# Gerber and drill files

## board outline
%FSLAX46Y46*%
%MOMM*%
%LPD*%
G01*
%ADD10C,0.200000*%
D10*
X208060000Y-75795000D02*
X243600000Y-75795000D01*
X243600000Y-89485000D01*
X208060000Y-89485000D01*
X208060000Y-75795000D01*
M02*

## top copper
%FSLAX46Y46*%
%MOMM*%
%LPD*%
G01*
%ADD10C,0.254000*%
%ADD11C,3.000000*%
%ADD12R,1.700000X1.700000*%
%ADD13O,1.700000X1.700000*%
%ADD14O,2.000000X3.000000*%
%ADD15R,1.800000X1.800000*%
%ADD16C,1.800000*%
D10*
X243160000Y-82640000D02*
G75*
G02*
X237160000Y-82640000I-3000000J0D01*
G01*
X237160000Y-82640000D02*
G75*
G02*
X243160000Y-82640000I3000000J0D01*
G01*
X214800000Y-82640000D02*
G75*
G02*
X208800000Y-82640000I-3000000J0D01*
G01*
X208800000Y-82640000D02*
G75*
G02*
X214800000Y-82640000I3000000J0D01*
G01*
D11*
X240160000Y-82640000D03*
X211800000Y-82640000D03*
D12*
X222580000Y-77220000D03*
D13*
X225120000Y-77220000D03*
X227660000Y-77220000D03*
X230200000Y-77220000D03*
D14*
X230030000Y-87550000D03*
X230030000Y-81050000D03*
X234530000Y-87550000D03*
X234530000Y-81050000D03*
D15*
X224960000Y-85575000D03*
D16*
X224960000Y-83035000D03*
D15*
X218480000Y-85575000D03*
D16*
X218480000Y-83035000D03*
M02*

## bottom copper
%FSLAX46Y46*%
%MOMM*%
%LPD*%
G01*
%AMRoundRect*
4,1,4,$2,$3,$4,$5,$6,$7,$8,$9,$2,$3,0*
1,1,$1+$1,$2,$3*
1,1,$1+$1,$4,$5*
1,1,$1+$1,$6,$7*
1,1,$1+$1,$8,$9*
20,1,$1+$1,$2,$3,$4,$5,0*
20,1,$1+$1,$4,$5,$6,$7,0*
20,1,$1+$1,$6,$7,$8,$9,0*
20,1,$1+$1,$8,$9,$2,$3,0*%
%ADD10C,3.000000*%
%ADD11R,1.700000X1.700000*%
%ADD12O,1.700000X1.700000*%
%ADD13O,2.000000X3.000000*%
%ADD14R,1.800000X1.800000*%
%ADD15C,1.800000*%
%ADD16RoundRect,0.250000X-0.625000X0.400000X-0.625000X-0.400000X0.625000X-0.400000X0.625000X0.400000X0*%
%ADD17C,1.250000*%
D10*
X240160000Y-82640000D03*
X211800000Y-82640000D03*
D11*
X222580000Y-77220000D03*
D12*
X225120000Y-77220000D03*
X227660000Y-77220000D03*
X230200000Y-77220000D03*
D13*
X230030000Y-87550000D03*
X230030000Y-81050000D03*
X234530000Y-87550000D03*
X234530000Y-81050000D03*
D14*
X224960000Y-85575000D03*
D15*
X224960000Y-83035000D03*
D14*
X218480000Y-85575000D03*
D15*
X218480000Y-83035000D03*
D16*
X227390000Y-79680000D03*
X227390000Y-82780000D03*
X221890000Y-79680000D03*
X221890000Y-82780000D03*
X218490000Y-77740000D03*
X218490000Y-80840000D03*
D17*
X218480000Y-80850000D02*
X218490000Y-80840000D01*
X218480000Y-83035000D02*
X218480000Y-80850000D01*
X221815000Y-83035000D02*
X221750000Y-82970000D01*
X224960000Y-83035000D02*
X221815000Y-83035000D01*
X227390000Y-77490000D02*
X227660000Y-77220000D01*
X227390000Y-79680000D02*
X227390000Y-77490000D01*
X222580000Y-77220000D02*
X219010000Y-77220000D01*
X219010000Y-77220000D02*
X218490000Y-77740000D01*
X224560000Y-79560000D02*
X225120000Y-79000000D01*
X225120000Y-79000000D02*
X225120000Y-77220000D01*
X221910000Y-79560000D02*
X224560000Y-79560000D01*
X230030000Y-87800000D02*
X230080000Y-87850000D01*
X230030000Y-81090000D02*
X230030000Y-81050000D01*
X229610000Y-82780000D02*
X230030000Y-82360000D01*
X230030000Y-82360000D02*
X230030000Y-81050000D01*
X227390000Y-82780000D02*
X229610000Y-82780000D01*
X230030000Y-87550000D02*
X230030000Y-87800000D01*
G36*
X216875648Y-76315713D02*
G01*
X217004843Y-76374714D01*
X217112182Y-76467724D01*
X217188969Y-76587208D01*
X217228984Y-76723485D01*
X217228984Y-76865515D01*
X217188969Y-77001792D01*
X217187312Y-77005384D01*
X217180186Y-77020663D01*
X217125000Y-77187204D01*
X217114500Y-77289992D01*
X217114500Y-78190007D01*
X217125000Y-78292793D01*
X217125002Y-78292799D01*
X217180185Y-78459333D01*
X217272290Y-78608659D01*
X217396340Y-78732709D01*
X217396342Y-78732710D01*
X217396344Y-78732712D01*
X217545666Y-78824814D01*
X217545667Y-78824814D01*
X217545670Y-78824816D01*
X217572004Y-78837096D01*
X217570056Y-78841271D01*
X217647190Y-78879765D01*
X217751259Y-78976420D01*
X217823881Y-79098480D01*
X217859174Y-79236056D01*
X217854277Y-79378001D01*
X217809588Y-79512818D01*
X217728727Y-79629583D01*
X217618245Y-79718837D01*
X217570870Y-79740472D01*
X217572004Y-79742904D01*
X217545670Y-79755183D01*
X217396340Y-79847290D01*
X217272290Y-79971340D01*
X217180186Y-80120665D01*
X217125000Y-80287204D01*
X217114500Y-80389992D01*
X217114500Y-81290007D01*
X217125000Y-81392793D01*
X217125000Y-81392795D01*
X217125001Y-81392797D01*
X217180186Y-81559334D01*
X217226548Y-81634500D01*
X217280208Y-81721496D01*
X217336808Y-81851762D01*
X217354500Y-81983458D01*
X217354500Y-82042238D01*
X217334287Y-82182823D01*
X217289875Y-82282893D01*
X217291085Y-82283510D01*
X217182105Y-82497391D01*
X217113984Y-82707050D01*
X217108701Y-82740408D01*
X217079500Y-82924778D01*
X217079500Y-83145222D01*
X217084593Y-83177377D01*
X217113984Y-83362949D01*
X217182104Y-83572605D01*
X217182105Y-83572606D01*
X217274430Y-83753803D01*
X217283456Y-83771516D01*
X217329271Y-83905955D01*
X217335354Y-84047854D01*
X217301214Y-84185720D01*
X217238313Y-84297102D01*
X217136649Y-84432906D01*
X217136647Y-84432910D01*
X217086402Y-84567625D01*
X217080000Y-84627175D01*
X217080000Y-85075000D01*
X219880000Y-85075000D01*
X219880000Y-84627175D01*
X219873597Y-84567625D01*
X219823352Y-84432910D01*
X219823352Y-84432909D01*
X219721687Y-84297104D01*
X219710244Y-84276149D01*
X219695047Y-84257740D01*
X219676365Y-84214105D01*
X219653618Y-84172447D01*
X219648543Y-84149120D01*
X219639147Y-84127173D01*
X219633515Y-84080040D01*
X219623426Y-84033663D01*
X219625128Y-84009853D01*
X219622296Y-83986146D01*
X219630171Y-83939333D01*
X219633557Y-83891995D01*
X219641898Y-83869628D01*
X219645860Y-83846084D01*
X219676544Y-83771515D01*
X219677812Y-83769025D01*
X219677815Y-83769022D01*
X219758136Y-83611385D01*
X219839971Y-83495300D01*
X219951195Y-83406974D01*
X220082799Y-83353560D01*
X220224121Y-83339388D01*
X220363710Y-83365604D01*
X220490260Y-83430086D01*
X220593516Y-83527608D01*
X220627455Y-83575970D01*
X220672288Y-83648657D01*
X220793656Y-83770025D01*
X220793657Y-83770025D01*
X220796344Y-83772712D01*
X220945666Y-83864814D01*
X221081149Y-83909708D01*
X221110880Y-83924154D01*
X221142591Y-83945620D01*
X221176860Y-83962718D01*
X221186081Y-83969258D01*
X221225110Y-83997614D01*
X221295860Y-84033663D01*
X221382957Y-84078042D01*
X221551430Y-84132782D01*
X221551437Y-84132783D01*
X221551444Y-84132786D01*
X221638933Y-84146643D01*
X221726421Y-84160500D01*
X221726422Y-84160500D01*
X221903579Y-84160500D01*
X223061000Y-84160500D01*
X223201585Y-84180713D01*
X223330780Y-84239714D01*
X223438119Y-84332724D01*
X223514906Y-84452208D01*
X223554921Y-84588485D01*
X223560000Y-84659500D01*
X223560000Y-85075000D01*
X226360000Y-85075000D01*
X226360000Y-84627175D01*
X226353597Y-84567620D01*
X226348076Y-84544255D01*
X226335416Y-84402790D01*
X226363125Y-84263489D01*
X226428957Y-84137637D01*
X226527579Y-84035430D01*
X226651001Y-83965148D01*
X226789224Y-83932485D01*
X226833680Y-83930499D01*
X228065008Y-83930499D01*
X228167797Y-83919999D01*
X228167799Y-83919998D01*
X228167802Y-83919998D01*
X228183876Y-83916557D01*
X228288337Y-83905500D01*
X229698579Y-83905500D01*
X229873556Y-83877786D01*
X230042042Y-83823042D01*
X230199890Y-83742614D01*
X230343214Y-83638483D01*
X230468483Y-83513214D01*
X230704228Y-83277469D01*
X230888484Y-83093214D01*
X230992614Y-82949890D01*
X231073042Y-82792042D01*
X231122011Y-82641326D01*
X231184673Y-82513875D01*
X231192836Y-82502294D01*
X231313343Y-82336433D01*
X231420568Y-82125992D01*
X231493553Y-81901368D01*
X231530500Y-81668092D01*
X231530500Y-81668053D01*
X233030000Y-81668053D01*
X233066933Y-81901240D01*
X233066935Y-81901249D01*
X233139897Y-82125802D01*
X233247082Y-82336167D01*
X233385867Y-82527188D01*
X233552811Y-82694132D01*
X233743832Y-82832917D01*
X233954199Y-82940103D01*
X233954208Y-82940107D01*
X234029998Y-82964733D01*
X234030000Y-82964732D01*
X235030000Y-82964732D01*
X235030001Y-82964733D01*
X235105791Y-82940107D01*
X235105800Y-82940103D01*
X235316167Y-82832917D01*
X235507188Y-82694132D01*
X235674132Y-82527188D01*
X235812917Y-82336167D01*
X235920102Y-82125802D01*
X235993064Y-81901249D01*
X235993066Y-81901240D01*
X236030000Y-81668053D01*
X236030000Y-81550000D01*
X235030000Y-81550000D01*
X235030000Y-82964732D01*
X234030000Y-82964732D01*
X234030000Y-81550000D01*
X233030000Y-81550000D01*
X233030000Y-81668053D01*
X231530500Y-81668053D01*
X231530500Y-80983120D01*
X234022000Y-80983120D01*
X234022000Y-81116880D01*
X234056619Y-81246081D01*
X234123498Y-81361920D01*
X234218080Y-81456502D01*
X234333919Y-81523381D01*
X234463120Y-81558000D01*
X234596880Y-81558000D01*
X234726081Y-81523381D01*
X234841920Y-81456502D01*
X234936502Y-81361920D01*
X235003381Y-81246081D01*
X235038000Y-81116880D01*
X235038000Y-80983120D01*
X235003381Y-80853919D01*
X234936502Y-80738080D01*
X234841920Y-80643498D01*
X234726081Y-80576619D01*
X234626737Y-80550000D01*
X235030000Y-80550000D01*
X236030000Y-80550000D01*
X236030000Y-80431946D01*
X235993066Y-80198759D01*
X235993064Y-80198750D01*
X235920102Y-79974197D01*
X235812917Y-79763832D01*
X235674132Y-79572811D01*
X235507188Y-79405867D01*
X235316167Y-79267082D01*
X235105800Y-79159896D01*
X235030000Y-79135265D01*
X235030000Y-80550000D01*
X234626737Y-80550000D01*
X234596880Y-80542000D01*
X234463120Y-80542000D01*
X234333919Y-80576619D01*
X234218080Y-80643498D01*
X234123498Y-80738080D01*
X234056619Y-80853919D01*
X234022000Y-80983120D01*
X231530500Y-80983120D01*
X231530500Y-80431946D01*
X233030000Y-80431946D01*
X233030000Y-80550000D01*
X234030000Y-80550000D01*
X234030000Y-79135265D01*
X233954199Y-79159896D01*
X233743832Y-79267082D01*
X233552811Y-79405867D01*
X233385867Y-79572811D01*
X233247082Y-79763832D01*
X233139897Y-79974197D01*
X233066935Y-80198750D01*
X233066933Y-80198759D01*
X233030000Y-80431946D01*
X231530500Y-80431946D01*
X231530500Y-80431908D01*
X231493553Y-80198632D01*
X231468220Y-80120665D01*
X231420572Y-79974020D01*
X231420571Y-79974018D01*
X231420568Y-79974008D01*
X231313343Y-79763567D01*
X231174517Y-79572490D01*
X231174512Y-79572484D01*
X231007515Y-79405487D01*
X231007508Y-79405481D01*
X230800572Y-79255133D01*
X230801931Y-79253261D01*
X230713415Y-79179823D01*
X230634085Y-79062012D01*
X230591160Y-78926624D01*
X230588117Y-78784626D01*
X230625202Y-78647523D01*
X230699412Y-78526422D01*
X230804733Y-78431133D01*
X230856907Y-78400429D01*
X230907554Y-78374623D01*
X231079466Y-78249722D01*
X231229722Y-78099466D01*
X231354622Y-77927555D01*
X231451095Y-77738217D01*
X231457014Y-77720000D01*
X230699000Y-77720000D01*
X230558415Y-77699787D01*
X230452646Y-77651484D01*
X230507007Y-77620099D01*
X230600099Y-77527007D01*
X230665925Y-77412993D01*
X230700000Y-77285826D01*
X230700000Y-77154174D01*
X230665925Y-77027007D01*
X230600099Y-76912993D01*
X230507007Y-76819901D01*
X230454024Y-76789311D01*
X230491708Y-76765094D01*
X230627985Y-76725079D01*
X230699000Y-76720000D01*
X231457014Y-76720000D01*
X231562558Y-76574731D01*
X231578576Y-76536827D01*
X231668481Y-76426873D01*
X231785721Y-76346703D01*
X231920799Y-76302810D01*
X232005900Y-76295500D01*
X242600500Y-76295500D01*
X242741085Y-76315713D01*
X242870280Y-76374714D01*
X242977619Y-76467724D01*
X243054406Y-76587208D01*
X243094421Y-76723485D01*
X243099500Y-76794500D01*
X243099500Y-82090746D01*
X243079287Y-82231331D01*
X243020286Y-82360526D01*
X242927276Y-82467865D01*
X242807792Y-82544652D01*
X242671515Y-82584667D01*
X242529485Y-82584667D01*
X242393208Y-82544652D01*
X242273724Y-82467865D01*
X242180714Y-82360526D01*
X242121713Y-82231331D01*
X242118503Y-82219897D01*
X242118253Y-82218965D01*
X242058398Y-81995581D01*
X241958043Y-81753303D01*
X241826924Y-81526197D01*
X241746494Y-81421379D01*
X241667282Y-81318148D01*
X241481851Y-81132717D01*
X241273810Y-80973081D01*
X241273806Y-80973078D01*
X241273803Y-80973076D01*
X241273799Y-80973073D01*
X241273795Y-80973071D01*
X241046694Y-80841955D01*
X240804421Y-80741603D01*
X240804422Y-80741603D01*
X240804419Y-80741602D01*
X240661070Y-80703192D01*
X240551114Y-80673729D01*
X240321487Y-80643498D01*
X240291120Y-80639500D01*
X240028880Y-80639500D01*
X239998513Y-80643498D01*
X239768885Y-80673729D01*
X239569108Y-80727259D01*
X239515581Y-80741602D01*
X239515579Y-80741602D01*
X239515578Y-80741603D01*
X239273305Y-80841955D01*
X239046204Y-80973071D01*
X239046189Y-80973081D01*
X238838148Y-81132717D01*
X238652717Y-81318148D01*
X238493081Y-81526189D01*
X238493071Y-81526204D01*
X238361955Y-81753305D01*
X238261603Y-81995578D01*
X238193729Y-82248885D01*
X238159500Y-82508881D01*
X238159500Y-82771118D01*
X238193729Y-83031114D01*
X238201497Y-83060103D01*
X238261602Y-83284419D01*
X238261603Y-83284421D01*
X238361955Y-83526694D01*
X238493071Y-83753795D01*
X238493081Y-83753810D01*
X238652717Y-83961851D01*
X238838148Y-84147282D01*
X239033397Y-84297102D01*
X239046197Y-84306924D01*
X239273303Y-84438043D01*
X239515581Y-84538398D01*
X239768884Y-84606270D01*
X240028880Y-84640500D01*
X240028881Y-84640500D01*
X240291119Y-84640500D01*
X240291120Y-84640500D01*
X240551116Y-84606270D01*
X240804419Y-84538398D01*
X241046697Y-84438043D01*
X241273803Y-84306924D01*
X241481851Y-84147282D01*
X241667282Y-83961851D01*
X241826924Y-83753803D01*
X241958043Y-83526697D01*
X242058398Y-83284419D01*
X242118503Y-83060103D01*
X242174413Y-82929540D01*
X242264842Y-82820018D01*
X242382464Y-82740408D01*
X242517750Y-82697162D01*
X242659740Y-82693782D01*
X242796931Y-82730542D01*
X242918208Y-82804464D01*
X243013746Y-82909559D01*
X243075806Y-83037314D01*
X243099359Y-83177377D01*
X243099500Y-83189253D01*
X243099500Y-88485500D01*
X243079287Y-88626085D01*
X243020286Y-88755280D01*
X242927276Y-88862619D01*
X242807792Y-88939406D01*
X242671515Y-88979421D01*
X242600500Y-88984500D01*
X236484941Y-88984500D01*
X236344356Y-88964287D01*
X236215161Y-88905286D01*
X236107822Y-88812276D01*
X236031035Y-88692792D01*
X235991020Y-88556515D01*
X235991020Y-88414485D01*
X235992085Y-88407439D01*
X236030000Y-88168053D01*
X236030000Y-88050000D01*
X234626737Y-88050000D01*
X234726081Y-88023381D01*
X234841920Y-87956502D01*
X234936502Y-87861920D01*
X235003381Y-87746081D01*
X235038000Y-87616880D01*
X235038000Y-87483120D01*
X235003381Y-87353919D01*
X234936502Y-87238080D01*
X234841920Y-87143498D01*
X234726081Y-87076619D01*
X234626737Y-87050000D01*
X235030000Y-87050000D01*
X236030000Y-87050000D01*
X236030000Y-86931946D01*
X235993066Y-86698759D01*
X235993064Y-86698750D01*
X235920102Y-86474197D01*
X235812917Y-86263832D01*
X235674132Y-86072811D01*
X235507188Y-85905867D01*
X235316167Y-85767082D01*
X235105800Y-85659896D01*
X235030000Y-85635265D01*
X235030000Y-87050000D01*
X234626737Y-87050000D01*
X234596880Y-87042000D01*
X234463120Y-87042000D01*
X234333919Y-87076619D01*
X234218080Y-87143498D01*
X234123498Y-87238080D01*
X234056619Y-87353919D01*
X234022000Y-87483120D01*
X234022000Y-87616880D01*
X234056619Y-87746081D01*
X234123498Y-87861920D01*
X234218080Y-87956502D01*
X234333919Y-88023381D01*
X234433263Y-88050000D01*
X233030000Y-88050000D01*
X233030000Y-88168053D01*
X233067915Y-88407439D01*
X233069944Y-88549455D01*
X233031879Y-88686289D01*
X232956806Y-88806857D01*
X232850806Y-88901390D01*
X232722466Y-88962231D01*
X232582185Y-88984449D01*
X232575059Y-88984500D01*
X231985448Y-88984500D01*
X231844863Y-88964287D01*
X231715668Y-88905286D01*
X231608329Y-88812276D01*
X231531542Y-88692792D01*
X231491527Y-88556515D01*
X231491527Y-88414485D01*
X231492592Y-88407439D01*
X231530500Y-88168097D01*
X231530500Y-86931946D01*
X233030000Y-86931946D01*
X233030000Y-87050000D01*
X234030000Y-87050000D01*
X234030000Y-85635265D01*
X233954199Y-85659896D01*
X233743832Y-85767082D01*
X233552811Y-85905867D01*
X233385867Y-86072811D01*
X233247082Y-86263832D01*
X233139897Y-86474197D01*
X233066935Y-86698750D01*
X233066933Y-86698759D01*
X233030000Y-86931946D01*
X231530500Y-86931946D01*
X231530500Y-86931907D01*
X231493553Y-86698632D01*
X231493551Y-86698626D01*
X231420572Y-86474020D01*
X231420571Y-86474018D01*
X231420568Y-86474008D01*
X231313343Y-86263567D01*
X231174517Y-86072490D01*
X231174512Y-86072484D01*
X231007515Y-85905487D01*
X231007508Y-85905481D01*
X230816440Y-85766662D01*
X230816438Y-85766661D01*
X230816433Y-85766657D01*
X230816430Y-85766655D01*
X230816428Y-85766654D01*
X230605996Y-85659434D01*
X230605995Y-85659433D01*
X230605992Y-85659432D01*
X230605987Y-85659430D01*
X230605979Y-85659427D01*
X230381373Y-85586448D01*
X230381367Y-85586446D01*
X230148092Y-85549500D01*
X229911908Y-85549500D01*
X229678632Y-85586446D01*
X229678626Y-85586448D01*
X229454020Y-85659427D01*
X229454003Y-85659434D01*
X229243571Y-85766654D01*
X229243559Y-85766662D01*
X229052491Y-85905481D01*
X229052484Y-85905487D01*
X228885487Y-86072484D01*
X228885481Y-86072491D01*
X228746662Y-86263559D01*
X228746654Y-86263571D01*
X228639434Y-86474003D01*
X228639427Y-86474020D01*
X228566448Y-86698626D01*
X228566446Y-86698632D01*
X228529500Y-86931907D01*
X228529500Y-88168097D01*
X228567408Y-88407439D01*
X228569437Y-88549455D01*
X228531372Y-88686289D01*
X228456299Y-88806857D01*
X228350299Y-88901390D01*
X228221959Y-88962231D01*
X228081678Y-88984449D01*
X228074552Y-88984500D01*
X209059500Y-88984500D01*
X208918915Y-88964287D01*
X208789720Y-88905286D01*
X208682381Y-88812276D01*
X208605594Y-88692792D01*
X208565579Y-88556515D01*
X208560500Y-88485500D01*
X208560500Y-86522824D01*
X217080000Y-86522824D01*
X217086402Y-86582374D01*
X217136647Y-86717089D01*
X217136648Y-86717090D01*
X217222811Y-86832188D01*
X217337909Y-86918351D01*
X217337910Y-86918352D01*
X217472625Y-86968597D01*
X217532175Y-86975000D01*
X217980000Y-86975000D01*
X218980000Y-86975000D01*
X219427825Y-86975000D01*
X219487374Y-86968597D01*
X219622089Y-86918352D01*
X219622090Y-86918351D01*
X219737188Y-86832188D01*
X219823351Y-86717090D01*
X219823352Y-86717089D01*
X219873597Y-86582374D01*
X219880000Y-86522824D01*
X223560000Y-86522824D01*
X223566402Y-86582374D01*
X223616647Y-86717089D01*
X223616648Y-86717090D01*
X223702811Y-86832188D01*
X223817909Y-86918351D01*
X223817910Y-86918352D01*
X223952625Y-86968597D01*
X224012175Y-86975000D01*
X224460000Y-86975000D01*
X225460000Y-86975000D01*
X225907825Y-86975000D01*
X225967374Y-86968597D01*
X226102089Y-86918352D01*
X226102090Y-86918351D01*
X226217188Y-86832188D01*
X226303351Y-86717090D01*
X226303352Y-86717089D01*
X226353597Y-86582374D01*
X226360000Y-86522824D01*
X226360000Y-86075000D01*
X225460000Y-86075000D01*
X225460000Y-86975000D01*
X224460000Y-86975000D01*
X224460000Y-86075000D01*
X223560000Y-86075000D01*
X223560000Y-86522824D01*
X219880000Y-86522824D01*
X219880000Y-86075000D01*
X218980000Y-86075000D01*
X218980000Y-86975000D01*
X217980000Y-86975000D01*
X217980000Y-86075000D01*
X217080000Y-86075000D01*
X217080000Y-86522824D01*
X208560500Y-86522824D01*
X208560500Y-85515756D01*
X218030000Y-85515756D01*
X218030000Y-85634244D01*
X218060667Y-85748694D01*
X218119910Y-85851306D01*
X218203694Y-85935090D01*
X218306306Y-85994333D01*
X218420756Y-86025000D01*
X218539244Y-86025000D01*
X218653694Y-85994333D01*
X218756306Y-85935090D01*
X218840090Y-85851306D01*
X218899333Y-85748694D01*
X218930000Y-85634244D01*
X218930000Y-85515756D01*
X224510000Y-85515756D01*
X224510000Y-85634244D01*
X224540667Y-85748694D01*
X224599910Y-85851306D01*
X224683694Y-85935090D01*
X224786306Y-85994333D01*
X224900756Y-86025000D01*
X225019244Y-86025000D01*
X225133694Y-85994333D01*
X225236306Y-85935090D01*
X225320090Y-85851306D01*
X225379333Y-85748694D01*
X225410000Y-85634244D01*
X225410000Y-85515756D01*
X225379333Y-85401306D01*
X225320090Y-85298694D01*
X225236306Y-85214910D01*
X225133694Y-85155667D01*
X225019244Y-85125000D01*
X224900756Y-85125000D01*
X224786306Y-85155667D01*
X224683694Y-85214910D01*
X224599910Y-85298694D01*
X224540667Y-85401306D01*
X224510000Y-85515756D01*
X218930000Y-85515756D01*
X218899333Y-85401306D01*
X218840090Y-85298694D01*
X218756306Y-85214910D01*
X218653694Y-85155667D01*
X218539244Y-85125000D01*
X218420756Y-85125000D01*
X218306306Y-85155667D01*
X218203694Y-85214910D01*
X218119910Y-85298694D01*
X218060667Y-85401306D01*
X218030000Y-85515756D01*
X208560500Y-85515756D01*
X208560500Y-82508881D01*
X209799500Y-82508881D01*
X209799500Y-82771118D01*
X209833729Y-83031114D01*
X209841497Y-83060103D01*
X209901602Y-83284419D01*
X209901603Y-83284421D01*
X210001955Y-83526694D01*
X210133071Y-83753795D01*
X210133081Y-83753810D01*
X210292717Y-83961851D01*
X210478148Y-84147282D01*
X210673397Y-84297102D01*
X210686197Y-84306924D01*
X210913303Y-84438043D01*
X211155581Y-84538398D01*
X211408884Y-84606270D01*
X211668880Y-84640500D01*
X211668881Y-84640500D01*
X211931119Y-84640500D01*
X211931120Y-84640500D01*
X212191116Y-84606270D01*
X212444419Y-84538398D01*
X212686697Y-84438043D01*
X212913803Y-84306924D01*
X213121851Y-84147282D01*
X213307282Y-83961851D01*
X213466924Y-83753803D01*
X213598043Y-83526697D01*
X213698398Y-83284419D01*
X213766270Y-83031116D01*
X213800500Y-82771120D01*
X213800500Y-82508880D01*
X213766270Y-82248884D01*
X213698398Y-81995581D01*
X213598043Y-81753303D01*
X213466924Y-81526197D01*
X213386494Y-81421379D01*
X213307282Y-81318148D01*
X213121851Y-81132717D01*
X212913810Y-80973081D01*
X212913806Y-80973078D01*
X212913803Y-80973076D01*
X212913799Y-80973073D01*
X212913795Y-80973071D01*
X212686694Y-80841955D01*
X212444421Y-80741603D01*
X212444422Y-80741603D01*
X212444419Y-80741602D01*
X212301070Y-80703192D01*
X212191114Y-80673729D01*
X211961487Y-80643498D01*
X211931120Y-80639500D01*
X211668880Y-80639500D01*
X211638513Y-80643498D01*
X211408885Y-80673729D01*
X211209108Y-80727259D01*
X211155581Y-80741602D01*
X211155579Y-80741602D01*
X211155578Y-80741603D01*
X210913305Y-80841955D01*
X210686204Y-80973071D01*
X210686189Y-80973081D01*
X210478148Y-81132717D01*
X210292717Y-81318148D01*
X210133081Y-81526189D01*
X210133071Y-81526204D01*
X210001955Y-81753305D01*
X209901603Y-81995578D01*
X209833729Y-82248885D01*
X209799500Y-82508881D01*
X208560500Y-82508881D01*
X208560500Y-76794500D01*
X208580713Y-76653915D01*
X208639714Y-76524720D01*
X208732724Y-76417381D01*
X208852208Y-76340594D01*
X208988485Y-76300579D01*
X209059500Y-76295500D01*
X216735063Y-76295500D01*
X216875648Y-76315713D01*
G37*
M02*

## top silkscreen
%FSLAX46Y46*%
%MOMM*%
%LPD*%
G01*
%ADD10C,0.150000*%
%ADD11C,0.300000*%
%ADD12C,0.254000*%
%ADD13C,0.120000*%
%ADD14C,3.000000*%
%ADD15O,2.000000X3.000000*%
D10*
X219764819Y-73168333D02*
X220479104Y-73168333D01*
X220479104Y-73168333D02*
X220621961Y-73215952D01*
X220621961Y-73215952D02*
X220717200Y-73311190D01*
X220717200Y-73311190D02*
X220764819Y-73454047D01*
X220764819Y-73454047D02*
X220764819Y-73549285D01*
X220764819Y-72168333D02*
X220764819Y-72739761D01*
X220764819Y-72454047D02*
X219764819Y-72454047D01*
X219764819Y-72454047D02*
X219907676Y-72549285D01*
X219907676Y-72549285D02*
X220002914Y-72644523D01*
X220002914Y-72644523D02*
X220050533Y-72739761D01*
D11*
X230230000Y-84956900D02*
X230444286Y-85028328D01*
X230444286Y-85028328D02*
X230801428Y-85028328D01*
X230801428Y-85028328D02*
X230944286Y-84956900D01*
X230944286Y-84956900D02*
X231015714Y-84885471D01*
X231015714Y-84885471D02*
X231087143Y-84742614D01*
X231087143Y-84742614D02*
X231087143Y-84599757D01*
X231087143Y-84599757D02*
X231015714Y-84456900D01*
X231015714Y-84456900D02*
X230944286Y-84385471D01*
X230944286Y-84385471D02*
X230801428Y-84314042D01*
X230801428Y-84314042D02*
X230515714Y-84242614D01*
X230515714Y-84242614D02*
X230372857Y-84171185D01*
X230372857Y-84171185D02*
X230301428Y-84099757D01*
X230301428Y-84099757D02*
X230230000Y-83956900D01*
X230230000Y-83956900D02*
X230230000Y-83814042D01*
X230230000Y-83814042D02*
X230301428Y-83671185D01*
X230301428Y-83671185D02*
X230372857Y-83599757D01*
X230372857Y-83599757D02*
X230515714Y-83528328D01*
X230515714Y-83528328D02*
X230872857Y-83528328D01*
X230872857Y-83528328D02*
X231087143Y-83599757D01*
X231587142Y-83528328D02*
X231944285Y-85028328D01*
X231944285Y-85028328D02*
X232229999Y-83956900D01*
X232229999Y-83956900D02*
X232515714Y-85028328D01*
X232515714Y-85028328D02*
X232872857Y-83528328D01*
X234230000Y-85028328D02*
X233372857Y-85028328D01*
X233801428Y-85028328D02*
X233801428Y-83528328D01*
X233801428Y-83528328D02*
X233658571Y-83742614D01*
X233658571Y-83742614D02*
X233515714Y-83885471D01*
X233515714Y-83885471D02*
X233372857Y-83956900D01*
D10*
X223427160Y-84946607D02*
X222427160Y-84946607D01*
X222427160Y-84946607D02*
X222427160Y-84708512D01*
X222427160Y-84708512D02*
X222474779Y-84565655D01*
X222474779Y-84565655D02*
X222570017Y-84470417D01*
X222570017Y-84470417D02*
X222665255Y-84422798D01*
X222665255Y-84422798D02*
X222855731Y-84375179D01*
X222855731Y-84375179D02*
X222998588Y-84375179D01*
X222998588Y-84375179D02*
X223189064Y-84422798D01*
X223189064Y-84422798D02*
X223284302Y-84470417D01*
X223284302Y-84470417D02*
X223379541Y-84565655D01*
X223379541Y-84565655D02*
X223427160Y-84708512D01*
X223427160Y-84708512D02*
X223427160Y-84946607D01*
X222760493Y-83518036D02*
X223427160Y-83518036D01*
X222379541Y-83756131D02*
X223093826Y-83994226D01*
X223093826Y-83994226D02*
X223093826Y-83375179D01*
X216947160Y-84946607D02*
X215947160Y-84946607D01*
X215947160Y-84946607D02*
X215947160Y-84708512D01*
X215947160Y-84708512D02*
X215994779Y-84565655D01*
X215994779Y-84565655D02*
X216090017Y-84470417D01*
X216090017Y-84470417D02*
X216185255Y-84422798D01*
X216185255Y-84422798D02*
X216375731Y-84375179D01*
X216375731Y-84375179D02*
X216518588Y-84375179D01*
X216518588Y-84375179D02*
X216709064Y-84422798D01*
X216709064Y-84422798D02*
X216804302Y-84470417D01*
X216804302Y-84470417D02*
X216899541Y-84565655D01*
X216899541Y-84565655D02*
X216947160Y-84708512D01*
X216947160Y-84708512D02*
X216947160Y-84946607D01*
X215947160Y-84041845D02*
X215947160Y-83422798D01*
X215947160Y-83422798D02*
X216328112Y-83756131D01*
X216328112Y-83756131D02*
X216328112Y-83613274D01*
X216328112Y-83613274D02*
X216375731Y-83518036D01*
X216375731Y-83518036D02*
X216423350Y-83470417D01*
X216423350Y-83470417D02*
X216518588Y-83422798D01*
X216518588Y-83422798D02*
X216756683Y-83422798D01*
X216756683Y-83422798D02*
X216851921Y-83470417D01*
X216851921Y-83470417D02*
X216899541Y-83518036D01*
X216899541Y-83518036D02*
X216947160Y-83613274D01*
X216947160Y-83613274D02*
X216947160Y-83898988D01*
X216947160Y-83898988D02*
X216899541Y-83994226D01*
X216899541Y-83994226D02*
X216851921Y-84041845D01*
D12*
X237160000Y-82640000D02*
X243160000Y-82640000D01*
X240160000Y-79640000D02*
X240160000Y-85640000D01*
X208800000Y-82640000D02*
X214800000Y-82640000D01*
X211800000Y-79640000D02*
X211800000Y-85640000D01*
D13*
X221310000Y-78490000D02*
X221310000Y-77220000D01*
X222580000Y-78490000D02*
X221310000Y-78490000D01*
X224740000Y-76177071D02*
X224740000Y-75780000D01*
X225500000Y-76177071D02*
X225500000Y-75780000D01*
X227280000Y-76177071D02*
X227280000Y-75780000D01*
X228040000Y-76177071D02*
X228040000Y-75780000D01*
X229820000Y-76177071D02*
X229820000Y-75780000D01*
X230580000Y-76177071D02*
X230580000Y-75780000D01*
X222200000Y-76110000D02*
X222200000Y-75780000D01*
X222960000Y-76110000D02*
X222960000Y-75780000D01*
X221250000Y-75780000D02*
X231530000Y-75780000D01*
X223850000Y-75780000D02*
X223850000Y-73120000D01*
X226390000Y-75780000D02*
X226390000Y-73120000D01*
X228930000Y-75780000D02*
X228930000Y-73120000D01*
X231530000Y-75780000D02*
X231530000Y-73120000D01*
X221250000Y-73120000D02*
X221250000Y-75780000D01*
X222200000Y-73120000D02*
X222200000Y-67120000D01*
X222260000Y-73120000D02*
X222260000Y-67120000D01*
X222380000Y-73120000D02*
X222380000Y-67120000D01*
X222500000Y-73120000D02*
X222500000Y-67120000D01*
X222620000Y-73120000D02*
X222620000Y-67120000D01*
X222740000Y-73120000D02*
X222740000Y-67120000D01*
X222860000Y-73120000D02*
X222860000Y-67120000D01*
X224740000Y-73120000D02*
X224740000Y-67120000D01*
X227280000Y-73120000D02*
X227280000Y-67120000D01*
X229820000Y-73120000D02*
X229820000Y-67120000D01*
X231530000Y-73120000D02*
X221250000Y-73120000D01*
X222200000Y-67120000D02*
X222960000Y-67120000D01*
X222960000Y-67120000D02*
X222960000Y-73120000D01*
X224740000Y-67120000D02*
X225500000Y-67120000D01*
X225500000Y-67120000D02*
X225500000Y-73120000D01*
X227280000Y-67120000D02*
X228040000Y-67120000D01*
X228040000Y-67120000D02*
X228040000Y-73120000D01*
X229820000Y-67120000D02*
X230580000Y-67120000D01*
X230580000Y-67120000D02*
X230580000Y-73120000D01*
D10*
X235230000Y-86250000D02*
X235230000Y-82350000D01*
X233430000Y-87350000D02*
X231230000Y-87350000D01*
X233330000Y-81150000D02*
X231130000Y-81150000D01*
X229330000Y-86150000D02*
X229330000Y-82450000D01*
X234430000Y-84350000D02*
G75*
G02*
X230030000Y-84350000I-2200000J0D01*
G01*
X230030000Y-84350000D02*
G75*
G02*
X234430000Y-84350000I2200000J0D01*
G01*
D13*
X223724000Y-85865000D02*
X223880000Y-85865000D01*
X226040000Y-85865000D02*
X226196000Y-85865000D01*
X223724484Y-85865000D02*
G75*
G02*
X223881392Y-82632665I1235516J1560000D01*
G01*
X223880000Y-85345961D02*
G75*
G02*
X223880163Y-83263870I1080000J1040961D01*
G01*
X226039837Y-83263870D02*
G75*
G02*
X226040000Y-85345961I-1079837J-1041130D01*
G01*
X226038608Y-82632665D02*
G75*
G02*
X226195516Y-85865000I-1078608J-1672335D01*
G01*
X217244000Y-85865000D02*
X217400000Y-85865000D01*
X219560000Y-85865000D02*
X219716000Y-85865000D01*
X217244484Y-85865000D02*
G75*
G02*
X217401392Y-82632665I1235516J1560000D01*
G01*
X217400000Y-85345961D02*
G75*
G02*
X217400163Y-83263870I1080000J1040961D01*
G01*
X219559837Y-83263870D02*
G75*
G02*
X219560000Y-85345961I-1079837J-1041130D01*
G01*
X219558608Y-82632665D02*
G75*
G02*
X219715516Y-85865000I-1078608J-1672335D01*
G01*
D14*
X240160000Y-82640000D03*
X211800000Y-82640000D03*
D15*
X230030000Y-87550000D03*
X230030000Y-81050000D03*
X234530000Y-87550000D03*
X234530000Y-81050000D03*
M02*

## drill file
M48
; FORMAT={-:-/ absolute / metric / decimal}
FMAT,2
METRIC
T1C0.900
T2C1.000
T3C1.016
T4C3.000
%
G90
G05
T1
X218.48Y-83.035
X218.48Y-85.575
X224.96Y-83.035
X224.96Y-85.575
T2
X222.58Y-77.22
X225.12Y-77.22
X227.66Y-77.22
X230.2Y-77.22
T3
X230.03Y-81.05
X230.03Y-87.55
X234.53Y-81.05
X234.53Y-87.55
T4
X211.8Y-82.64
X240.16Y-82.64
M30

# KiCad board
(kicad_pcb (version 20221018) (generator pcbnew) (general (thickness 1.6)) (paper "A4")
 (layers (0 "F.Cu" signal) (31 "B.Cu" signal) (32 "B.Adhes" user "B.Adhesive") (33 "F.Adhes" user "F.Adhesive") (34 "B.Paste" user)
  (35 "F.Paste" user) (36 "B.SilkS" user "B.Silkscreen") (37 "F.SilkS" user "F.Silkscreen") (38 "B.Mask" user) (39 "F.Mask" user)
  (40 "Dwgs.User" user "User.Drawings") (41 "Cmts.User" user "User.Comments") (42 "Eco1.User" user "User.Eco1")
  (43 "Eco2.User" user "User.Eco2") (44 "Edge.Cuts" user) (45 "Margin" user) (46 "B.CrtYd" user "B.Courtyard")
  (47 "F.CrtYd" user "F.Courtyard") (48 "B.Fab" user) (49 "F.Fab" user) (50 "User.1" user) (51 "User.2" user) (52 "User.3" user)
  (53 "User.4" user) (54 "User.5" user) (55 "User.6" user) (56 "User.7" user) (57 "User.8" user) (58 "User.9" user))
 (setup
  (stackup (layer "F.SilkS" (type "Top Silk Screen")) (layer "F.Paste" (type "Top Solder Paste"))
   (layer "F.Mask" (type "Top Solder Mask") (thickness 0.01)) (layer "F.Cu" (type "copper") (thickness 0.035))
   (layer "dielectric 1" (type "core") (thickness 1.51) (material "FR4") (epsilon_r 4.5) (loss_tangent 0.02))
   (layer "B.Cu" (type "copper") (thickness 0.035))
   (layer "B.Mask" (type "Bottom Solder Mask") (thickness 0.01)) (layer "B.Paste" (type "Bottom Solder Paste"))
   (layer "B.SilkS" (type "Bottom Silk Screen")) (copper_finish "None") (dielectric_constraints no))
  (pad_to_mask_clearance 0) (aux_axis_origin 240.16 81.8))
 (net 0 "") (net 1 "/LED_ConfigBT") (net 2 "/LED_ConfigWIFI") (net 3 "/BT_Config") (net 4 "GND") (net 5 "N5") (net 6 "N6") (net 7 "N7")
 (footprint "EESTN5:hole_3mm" (layer "F.Cu") (at 240.16 82.64)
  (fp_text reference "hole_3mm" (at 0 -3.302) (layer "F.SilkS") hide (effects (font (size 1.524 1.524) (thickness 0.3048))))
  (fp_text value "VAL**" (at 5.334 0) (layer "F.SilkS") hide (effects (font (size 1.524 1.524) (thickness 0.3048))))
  (fp_circle (center 0 0) (end 3 0) (stroke (width 0.254) (type solid)) (fill none) (layer "F.Cu"))
  (fp_line (start -3 0) (end 3 0) (stroke (width 0.254) (type solid)) (layer "F.SilkS"))
  (fp_line (start 0 -3) (end 0 3) (stroke (width 0.254) (type solid)) (layer "F.SilkS"))
  (pad "1" thru_hole circle (at 0 0) (size 3 3) (drill 3) (layers "*.Cu" "F.SilkS")))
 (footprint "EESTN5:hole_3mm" (layer "F.Cu") (at 211.8 82.64)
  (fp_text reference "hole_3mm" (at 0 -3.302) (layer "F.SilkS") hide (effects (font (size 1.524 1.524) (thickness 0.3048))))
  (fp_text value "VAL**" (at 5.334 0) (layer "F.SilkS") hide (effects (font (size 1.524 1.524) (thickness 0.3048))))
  (fp_circle (center 0 0) (end 3 0) (stroke (width 0.254) (type solid)) (fill none) (layer "F.Cu"))
  (fp_line (start -3 0) (end 3 0) (stroke (width 0.254) (type solid)) (layer "F.SilkS"))
  (fp_line (start 0 -3) (end 0 3) (stroke (width 0.254) (type solid)) (layer "F.SilkS"))
  (pad "1" thru_hole circle (at 0 0) (size 3 3) (drill 3) (layers "*.Cu" "F.SilkS")))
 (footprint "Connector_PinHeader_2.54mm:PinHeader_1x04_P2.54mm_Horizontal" (layer "F.Cu") (at 222.58 77.22 90)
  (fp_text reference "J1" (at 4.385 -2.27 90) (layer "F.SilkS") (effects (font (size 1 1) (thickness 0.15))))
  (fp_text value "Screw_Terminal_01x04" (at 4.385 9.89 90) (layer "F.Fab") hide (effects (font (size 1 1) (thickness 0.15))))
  (fp_line (start -1.27 -1.27) (end 0 -1.27) (stroke (width 0.12) (type solid)) (layer "F.SilkS"))
  (fp_line (start -1.27 0) (end -1.27 -1.27) (stroke (width 0.12) (type solid)) (layer "F.SilkS"))
  (fp_line (start 1.042929 2.16) (end 1.44 2.16) (stroke (width 0.12) (type solid)) (layer "F.SilkS"))
  (fp_line (start 1.042929 2.92) (end 1.44 2.92) (stroke (width 0.12) (type solid)) (layer "F.SilkS"))
  (fp_line (start 1.042929 4.7) (end 1.44 4.7) (stroke (width 0.12) (type solid)) (layer "F.SilkS"))
  (fp_line (start 1.042929 5.46) (end 1.44 5.46) (stroke (width 0.12) (type solid)) (layer "F.SilkS"))
  (fp_line (start 1.042929 7.24) (end 1.44 7.24) (stroke (width 0.12) (type solid)) (layer "F.SilkS"))
  (fp_line (start 1.042929 8) (end 1.44 8) (stroke (width 0.12) (type solid)) (layer "F.SilkS"))
  (fp_line (start 1.11 -0.38) (end 1.44 -0.38) (stroke (width 0.12) (type solid)) (layer "F.SilkS"))
  (fp_line (start 1.11 0.38) (end 1.44 0.38) (stroke (width 0.12) (type solid)) (layer "F.SilkS"))
  (fp_line (start 1.44 -1.33) (end 1.44 8.95) (stroke (width 0.12) (type solid)) (layer "F.SilkS"))
  (fp_line (start 1.44 1.27) (end 4.1 1.27) (stroke (width 0.12) (type solid)) (layer "F.SilkS"))
  (fp_line (start 1.44 3.81) (end 4.1 3.81) (stroke (width 0.12) (type solid)) (layer "F.SilkS"))
  (fp_line (start 1.44 6.35) (end 4.1 6.35) (stroke (width 0.12) (type solid)) (layer "F.SilkS"))
  (fp_line (start 1.44 8.95) (end 4.1 8.95) (stroke (width 0.12) (type solid)) (layer "F.SilkS"))
  (fp_line (start 4.1 -1.33) (end 1.44 -1.33) (stroke (width 0.12) (type solid)) (layer "F.SilkS"))
  (fp_line (start 4.1 -0.38) (end 10.1 -0.38) (stroke (width 0.12) (type solid)) (layer "F.SilkS"))
  (fp_line (start 4.1 -0.32) (end 10.1 -0.32) (stroke (width 0.12) (type solid)) (layer "F.SilkS"))
  (fp_line (start 4.1 -0.2) (end 10.1 -0.2) (stroke (width 0.12) (type solid)) (layer "F.SilkS"))
  (fp_line (start 4.1 -0.08) (end 10.1 -0.08) (stroke (width 0.12) (type solid)) (layer "F.SilkS"))
  (fp_line (start 4.1 0.04) (end 10.1 0.04) (stroke (width 0.12) (type solid)) (layer "F.SilkS"))
  (fp_line (start 4.1 0.16) (end 10.1 0.16) (stroke (width 0.12) (type solid)) (layer "F.SilkS"))
  (fp_line (start 4.1 0.28) (end 10.1 0.28) (stroke (width 0.12) (type solid)) (layer "F.SilkS"))
  (fp_line (start 4.1 2.16) (end 10.1 2.16) (stroke (width 0.12) (type solid)) (layer "F.SilkS"))
  (fp_line (start 4.1 4.7) (end 10.1 4.7) (stroke (width 0.12) (type solid)) (layer "F.SilkS"))
  (fp_line (start 4.1 7.24) (end 10.1 7.24) (stroke (width 0.12) (type solid)) (layer "F.SilkS"))
  (fp_line (start 4.1 8.95) (end 4.1 -1.33) (stroke (width 0.12) (type solid)) (layer "F.SilkS"))
  (fp_line (start 10.1 -0.38) (end 10.1 0.38) (stroke (width 0.12) (type solid)) (layer "F.SilkS"))
  (fp_line (start 10.1 0.38) (end 4.1 0.38) (stroke (width 0.12) (type solid)) (layer "F.SilkS"))
  (fp_line (start 10.1 2.16) (end 10.1 2.92) (stroke (width 0.12) (type solid)) (layer "F.SilkS"))
  (fp_line (start 10.1 2.92) (end 4.1 2.92) (stroke (width 0.12) (type solid)) (layer "F.SilkS"))
  (fp_line (start 10.1 4.7) (end 10.1 5.46) (stroke (width 0.12) (type solid)) (layer "F.SilkS"))
  (fp_line (start 10.1 5.46) (end 4.1 5.46) (stroke (width 0.12) (type solid)) (layer "F.SilkS"))
  (fp_line (start 10.1 7.24) (end 10.1 8) (stroke (width 0.12) (type solid)) (layer "F.SilkS"))
  (fp_line (start 10.1 8) (end 4.1 8) (stroke (width 0.12) (type solid)) (layer "F.SilkS"))
  (pad "1" thru_hole rect (at 0 0 90) (size 1.7 1.7) (drill 1) (layers "*.Cu" "*.Mask") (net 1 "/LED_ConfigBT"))
  (pad "2" thru_hole oval (at 0 2.54 90) (size 1.7 1.7) (drill 1) (layers "*.Cu" "*.Mask") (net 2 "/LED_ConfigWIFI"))
  (pad "3" thru_hole oval (at 0 5.08 90) (size 1.7 1.7) (drill 1) (layers "*.Cu" "*.Mask") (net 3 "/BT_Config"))
  (pad "4" thru_hole oval (at 0 7.62 90) (size 1.7 1.7) (drill 1) (layers "*.Cu" "*.Mask") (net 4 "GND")))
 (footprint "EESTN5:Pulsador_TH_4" (layer "F.Cu") (at 232.28 84.3 180)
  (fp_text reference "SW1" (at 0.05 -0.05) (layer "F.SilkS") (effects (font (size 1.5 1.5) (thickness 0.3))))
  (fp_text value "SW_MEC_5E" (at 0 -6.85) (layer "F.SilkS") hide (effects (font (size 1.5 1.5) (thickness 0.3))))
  (fp_line (start -2.95 -1.95) (end -2.95 1.95) (stroke (width 0.15) (type solid)) (layer "F.SilkS"))
  (fp_line (start -1.15 -3.05) (end 1.05 -3.05) (stroke (width 0.15) (type solid)) (layer "F.SilkS"))
  (fp_line (start -1.05 3.15) (end 1.15 3.15) (stroke (width 0.15) (type solid)) (layer "F.SilkS"))
  (fp_line (start 2.95 -1.85) (end 2.95 1.85) (stroke (width 0.15) (type solid)) (layer "F.SilkS"))
  (fp_circle (center 0.05 -0.05) (end 0.05 2.15) (stroke (width 0.15) (type solid)) (fill none) (layer "F.SilkS"))
  (pad "1" thru_hole oval (at 2.25 -3.25 180) (size 2 3) (drill 1.016) (layers "*.Cu" "*.Mask" "F.SilkS") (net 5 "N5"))
  (pad "2" thru_hole oval (at 2.25 3.25 180) (size 2 3) (drill 1.016) (layers "*.Cu" "*.Mask" "F.SilkS") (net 5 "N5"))
  (pad "3" thru_hole oval (at -2.25 -3.25 180) (size 2 3) (drill 1.016) (layers "*.Cu" "*.Mask" "F.SilkS") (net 4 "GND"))
  (pad "4" thru_hole oval (at -2.25 3.25 180) (size 2 3) (drill 1.016) (layers "*.Cu" "*.Mask" "F.SilkS") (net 4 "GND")))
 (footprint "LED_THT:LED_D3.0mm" (layer "F.Cu") (at 224.96 85.575 90)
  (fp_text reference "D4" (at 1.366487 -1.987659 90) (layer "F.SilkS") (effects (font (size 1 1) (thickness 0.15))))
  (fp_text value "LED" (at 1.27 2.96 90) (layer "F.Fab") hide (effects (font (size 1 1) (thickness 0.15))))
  (fp_line (start -0.29 -1.236) (end -0.29 -1.08) (stroke (width 0.12) (type solid)) (layer "F.SilkS"))
  (fp_line (start -0.29 1.08) (end -0.29 1.236) (stroke (width 0.12) (type solid)) (layer "F.SilkS"))
  (fp_arc (start -0.29 -1.235516) (mid 1.366487 -1.987659) (end 2.942335 -1.078608) (stroke (width 0.12) (type solid)) (layer "F.SilkS"))
  (fp_arc (start 0.229039 -1.08) (mid 1.270117 -1.5) (end 2.31113 -1.079837) (stroke (width 0.12) (type solid)) (layer "F.SilkS"))
  (fp_arc (start 2.31113 1.079837) (mid 1.270117 1.5) (end 0.229039 1.08) (stroke (width 0.12) (type solid)) (layer "F.SilkS"))
  (fp_arc (start 2.942335 1.078608) (mid 1.366487 1.987659) (end -0.29 1.235516) (stroke (width 0.12) (type solid)) (layer "F.SilkS"))
  (pad "1" thru_hole rect (at 0 0 90) (size 1.8 1.8) (drill 0.9) (layers "*.Cu" "*.Mask") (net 4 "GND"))
  (pad "2" thru_hole circle (at 2.54 0 90) (size 1.8 1.8) (drill 0.9) (layers "*.Cu" "*.Mask") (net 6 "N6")))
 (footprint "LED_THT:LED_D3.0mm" (layer "F.Cu") (at 218.48 85.575 90)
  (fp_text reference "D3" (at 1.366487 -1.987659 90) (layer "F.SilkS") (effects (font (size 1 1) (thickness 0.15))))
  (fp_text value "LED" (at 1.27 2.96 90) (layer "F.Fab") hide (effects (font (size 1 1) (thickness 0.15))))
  (fp_line (start -0.29 -1.236) (end -0.29 -1.08) (stroke (width 0.12) (type solid)) (layer "F.SilkS"))
  (fp_line (start -0.29 1.08) (end -0.29 1.236) (stroke (width 0.12) (type solid)) (layer "F.SilkS"))
  (fp_arc (start -0.29 -1.235516) (mid 1.366487 -1.987659) (end 2.942335 -1.078608) (stroke (width 0.12) (type solid)) (layer "F.SilkS"))
  (fp_arc (start 0.229039 -1.08) (mid 1.270117 -1.5) (end 2.31113 -1.079837) (stroke (width 0.12) (type solid)) (layer "F.SilkS"))
  (fp_arc (start 2.31113 1.079837) (mid 1.270117 1.5) (end 0.229039 1.08) (stroke (width 0.12) (type solid)) (layer "F.SilkS"))
  (fp_arc (start 2.942335 1.078608) (mid 1.366487 1.987659) (end -0.29 1.235516) (stroke (width 0.12) (type solid)) (layer "F.SilkS"))
  (pad "1" thru_hole rect (at 0 0 90) (size 1.8 1.8) (drill 0.9) (layers "*.Cu" "*.Mask") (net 4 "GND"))
  (pad "2" thru_hole circle (at 2.54 0 90) (size 1.8 1.8) (drill 0.9) (layers "*.Cu" "*.Mask") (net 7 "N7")))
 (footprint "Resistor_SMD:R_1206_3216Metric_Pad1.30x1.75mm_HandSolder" (layer "B.Cu") (at 227.39 81.23 -90)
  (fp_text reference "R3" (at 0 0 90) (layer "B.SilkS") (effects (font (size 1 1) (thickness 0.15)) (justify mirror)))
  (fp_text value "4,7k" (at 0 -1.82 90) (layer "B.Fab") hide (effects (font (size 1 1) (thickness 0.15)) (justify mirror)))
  (pad "1" smd roundrect (at -1.55 0 270) (size 1.3 1.75) (layers "B.Cu" "B.Paste" "B.Mask") (roundrect_rratio 0.192308)
   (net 3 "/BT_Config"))
  (pad "2" smd roundrect (at 1.55 0 270) (size 1.3 1.75) (layers "B.Cu" "B.Paste" "B.Mask") (roundrect_rratio 0.192308) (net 5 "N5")))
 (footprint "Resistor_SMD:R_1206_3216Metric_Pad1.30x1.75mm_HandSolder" (layer "B.Cu") (at 221.89 81.23 -90)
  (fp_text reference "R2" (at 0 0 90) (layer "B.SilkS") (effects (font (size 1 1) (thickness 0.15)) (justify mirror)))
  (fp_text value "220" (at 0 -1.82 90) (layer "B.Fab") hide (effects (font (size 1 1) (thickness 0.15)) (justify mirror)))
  (pad "1" smd roundrect (at -1.55 0 270) (size 1.3 1.75) (layers "B.Cu" "B.Paste" "B.Mask") (roundrect_rratio 0.192308)
   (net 2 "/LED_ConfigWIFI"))
  (pad "2" smd roundrect (at 1.55 0 270) (size 1.3 1.75) (layers "B.Cu" "B.Paste" "B.Mask") (roundrect_rratio 0.192308) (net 6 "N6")))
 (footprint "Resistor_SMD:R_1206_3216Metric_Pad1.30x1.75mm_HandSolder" (layer "B.Cu") (at 218.49 79.29 -90)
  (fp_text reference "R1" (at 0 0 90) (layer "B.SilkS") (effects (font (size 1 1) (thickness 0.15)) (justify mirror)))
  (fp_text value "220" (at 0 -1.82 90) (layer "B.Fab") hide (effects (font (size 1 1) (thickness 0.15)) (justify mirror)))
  (pad "1" smd roundrect (at -1.55 0 270) (size 1.3 1.75) (layers "B.Cu" "B.Paste" "B.Mask") (roundrect_rratio 0.192308)
   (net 1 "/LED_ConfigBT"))
  (pad "2" smd roundrect (at 1.55 0 270) (size 1.3 1.75) (layers "B.Cu" "B.Paste" "B.Mask") (roundrect_rratio 0.192308) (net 7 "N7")))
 (gr_rect (start 208.06 75.795) (end 243.6 89.485) (stroke (width 0.2) (type default)) (fill none) (layer "Edge.Cuts"))
 (segment (start 218.48 80.85) (end 218.49 80.84) (width 1.25) (layer "B.Cu") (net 7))
 (segment (start 218.48 83.035) (end 218.48 80.85) (width 1.25) (layer "B.Cu") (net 7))
 (segment (start 221.815 83.035) (end 221.75 82.97) (width 1.25) (layer "B.Cu") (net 6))
 (segment (start 224.96 83.035) (end 221.815 83.035) (width 1.25) (layer "B.Cu") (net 6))
 (segment (start 227.39 77.49) (end 227.66 77.22) (width 1.25) (layer "B.Cu") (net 3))
 (segment (start 227.39 79.68) (end 227.39 77.49) (width 1.25) (layer "B.Cu") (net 3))
 (segment (start 222.58 77.22) (end 219.01 77.22) (width 1.25) (layer "B.Cu") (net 1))
 (segment (start 219.01 77.22) (end 218.49 77.74) (width 1.25) (layer "B.Cu") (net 1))
 (segment (start 224.56 79.56) (end 225.12 79) (width 1.25) (layer "B.Cu") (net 2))
 (segment (start 225.12 79) (end 225.12 77.22) (width 1.25) (layer "B.Cu") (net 2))
 (segment (start 221.91 79.56) (end 224.56 79.56) (width 1.25) (layer "B.Cu") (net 2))
 (segment (start 230.03 87.8) (end 230.08 87.85) (width 1.25) (layer "B.Cu") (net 5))
 (segment (start 230.03 81.09) (end 230.03 81.05) (width 1.25) (layer "B.Cu") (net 5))
 (segment (start 229.61 82.78) (end 230.03 82.36) (width 1.25) (layer "B.Cu") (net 5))
 (segment (start 230.03 82.36) (end 230.03 81.05) (width 1.25) (layer "B.Cu") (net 5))
 (segment (start 227.39 82.78) (end 229.61 82.78) (width 1.25) (layer "B.Cu") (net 5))
 (segment (start 230.03 87.55) (end 230.03 87.8) (width 1.25) (layer "B.Cu") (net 5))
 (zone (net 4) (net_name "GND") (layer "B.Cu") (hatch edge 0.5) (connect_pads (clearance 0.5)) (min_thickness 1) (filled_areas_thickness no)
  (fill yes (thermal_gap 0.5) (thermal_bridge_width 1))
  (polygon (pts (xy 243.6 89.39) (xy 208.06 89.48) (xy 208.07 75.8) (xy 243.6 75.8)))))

